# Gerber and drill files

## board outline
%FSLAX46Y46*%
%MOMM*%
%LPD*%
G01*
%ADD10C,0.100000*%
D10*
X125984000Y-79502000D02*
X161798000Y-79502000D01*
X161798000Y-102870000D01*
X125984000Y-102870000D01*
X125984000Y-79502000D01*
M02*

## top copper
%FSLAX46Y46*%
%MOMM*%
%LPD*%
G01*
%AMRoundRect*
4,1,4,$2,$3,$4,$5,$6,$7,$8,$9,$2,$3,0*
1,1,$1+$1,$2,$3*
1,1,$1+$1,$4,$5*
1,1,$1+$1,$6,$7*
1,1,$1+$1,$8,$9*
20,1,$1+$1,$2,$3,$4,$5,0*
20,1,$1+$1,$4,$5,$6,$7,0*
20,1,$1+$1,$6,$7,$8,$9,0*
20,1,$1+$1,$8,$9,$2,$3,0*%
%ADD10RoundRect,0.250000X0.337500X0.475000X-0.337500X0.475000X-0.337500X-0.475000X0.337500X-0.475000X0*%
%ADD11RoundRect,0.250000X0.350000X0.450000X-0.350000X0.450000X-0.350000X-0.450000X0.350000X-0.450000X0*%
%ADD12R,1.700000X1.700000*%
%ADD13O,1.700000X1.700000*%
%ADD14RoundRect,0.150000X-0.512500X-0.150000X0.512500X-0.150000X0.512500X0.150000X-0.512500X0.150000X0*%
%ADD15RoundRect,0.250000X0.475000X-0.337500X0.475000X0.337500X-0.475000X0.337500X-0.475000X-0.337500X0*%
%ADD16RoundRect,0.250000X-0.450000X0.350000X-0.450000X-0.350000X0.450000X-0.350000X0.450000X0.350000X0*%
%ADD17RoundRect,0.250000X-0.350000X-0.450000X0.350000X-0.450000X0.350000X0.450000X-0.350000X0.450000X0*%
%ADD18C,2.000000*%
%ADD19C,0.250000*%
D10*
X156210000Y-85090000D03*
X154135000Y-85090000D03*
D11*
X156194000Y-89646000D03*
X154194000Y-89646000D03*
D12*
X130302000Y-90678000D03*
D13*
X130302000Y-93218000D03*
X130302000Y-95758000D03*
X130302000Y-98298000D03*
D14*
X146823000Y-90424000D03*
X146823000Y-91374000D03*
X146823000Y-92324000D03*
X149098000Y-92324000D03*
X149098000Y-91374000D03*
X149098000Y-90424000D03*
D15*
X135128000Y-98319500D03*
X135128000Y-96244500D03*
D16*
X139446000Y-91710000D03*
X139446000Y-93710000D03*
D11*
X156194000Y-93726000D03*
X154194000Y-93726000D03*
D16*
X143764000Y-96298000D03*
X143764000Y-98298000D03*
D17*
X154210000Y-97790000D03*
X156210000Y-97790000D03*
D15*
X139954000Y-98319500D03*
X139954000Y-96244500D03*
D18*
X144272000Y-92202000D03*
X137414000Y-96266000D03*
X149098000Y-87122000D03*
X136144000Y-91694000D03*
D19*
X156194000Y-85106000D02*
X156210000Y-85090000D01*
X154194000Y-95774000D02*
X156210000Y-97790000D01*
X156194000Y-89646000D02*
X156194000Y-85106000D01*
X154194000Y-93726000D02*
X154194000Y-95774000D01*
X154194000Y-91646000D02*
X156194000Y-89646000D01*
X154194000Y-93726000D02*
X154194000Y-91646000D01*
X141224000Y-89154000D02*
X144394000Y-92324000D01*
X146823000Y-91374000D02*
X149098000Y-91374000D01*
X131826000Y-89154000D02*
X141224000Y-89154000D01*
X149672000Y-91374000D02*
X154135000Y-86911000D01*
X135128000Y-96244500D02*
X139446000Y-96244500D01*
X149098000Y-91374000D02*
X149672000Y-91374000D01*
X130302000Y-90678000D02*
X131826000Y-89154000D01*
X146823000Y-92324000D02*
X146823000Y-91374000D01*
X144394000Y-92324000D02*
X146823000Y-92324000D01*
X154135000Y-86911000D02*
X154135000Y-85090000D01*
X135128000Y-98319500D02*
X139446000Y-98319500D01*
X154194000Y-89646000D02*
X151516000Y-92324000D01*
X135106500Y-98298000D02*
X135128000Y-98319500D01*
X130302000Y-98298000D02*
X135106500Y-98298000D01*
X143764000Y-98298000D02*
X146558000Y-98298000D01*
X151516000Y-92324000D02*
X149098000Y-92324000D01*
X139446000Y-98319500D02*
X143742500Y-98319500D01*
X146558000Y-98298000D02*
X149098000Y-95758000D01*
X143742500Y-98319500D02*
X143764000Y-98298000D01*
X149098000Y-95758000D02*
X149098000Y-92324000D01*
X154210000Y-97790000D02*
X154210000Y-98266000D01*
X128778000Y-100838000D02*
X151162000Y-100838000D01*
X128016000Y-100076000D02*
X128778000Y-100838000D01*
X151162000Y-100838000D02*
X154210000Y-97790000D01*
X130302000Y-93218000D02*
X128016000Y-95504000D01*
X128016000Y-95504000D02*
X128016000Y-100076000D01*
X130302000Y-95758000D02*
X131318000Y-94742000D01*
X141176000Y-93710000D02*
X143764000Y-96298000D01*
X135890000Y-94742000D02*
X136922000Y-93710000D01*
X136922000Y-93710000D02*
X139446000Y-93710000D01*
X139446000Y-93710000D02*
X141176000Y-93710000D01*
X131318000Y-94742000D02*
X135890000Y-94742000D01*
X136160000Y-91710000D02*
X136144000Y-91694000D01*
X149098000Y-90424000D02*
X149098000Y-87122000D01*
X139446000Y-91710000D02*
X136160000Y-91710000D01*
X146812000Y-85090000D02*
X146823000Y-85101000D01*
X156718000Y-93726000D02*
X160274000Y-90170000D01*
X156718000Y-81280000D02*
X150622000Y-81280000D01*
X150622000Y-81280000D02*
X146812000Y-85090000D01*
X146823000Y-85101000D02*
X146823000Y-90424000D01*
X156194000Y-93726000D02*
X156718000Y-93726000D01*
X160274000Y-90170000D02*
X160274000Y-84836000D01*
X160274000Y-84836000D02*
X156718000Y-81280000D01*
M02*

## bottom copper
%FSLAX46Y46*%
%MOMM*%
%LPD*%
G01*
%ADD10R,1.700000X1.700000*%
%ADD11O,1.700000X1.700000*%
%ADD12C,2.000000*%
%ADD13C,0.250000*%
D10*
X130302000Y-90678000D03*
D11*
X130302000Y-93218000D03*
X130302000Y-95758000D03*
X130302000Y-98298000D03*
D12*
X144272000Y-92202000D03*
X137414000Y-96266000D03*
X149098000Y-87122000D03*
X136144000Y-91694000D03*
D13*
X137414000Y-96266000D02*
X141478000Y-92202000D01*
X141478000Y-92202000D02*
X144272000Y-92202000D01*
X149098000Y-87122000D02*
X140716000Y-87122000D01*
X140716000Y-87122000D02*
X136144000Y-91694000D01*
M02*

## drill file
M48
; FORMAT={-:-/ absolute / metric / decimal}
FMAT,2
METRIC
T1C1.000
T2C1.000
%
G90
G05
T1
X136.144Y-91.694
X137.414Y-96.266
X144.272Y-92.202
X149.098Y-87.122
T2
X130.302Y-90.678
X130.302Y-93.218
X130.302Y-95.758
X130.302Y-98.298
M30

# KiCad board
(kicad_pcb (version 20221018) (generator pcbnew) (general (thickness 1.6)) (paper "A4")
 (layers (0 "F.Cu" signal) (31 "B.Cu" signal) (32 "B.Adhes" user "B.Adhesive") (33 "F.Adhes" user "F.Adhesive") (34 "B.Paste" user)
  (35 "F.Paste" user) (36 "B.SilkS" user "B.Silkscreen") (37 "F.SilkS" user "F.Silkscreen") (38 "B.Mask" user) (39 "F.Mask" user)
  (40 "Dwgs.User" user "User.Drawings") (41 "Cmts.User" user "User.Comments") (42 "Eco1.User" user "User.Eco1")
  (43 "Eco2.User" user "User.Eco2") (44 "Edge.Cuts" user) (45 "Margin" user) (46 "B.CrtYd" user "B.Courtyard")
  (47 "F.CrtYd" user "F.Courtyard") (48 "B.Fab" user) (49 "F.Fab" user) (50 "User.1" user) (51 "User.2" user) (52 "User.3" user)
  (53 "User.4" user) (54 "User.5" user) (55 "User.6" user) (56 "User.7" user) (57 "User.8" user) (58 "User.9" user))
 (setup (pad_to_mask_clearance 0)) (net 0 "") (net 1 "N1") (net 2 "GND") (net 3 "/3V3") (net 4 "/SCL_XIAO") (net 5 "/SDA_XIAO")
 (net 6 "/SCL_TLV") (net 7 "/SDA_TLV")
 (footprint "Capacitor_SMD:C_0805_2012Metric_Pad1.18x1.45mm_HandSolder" (layer "F.Cu") (at 155.1725 85.09 180)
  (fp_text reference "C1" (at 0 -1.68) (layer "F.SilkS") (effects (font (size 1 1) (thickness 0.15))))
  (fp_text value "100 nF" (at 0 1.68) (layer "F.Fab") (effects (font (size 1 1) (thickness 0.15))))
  (pad "1" smd roundrect (at -1.0375 0 180) (size 1.175 1.45) (layers "F.Cu" "F.Paste" "F.Mask") (roundrect_rratio 0.2127659574)
   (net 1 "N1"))
  (pad "2" smd roundrect (at 1.0375 0 180) (size 1.175 1.45) (layers "F.Cu" "F.Paste" "F.Mask") (roundrect_rratio 0.2127659574)
   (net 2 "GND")))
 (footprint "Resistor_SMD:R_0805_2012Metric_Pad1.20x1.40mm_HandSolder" (layer "F.Cu") (at 155.194 89.646 180)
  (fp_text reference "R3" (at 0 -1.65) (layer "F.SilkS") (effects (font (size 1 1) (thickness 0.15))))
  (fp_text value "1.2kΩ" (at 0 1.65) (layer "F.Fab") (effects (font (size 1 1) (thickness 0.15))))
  (pad "1" smd roundrect (at -1 0 180) (size 1.2 1.4) (layers "F.Cu" "F.Paste" "F.Mask") (roundrect_rratio 0.2083333333) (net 1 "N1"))
  (pad "2" smd roundrect (at 1 0 180) (size 1.2 1.4) (layers "F.Cu" "F.Paste" "F.Mask") (roundrect_rratio 0.2083333333) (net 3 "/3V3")))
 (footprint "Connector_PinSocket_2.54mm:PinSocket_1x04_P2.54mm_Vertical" (layer "F.Cu") (at 130.302 90.678)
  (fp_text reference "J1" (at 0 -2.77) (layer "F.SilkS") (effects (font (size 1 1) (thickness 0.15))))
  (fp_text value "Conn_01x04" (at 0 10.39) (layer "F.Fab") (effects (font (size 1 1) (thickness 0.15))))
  (pad "1" thru_hole rect (at 0 0) (size 1.7 1.7) (drill 1) (layers "*.Cu" "*.Mask") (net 2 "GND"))
  (pad "2" thru_hole oval (at 0 2.54) (size 1.7 1.7) (drill 1) (layers "*.Cu" "*.Mask") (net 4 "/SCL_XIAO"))
  (pad "3" thru_hole oval (at 0 5.08) (size 1.7 1.7) (drill 1) (layers "*.Cu" "*.Mask") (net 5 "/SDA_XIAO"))
  (pad "4" thru_hole oval (at 0 7.62) (size 1.7 1.7) (drill 1) (layers "*.Cu" "*.Mask") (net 3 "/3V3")))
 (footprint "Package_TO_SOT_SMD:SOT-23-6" (layer "F.Cu") (at 147.9605 91.374)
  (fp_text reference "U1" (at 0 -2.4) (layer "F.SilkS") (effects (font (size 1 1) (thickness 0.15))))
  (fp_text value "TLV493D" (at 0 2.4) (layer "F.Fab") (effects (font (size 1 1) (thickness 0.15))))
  (pad "1" smd roundrect (at -1.1375 -0.95) (size 1.325 0.6) (layers "F.Cu" "F.Paste" "F.Mask") (roundrect_rratio 0.25) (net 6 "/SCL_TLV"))
  (pad "2" smd roundrect (at -1.1375 0) (size 1.325 0.6) (layers "F.Cu" "F.Paste" "F.Mask") (roundrect_rratio 0.25) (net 2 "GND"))
  (pad "3" smd roundrect (at -1.1375 0.95) (size 1.325 0.6) (layers "F.Cu" "F.Paste" "F.Mask") (roundrect_rratio 0.25) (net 2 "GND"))
  (pad "4" smd roundrect (at 1.1375 0.95) (size 1.325 0.6) (layers "F.Cu" "F.Paste" "F.Mask") (roundrect_rratio 0.25) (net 3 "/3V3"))
  (pad "5" smd roundrect (at 1.1375 0) (size 1.325 0.6) (layers "F.Cu" "F.Paste" "F.Mask") (roundrect_rratio 0.25) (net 2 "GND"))
  (pad "6" smd roundrect (at 1.1375 -0.95) (size 1.325 0.6) (layers "F.Cu" "F.Paste" "F.Mask") (roundrect_rratio 0.25) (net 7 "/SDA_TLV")))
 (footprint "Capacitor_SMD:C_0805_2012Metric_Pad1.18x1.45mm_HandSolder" (layer "F.Cu") (at 135.128 97.282 90)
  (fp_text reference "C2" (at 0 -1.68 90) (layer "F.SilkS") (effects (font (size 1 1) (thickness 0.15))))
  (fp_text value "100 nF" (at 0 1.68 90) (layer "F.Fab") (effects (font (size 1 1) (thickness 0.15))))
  (pad "1" smd roundrect (at -1.0375 0 90) (size 1.175 1.45) (layers "F.Cu" "F.Paste" "F.Mask") (roundrect_rratio 0.2127659574)
   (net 3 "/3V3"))
  (pad "2" smd roundrect (at 1.0375 0 90) (size 1.175 1.45) (layers "F.Cu" "F.Paste" "F.Mask") (roundrect_rratio 0.2127659574) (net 2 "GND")))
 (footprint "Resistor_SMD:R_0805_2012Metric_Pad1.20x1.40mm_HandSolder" (layer "F.Cu") (at 139.446 92.71 -90)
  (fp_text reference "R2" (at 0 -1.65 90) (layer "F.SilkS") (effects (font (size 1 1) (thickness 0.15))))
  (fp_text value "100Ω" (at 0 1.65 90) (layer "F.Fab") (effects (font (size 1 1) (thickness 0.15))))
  (pad "1" smd roundrect (at -1 0 270) (size 1.2 1.4) (layers "F.Cu" "F.Paste" "F.Mask") (roundrect_rratio 0.2083333333) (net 7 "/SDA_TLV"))
  (pad "2" smd roundrect (at 1 0 270) (size 1.2 1.4) (layers "F.Cu" "F.Paste" "F.Mask") (roundrect_rratio 0.2083333333) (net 5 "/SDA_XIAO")))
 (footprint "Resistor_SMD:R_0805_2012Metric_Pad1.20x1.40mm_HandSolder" (layer "F.Cu") (at 155.194 93.726 180)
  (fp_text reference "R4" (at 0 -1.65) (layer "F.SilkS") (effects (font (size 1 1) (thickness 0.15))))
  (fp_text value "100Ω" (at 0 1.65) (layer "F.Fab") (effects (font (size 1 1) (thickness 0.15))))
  (pad "1" smd roundrect (at -1 0 180) (size 1.2 1.4) (layers "F.Cu" "F.Paste" "F.Mask") (roundrect_rratio 0.2083333333) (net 6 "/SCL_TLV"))
  (pad "2" smd roundrect (at 1 0 180) (size 1.2 1.4) (layers "F.Cu" "F.Paste" "F.Mask") (roundrect_rratio 0.2083333333) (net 1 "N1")))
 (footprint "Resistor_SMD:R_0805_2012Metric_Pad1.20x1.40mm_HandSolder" (layer "F.Cu") (at 143.764 97.298 -90)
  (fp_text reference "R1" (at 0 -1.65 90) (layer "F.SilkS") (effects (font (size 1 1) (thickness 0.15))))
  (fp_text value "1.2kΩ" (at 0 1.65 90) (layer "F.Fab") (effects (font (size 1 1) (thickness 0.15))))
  (pad "1" smd roundrect (at -1 0 270) (size 1.2 1.4) (layers "F.Cu" "F.Paste" "F.Mask") (roundrect_rratio 0.2083333333) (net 5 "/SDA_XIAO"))
  (pad "2" smd roundrect (at 1 0 270) (size 1.2 1.4) (layers "F.Cu" "F.Paste" "F.Mask") (roundrect_rratio 0.2083333333) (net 3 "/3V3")))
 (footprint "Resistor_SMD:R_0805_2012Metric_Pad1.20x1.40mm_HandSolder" (layer "F.Cu") (at 155.21 97.79)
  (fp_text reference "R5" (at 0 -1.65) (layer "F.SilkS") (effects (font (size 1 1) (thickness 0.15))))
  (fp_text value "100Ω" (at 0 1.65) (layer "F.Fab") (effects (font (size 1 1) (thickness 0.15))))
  (pad "1" smd roundrect (at -1 0) (size 1.2 1.4) (layers "F.Cu" "F.Paste" "F.Mask") (roundrect_rratio 0.2083333333) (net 4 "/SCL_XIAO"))
  (pad "2" smd roundrect (at 1 0) (size 1.2 1.4) (layers "F.Cu" "F.Paste" "F.Mask") (roundrect_rratio 0.2083333333) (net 1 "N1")))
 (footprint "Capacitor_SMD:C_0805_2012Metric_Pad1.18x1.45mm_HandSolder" (layer "F.Cu") (at 139.954 97.282 90)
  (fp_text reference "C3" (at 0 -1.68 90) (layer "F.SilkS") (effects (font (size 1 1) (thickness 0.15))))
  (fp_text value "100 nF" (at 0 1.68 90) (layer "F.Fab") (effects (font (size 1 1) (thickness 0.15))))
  (pad "1" smd roundrect (at -1.0375 0 90) (size 1.175 1.45) (layers "F.Cu" "F.Paste" "F.Mask") (roundrect_rratio 0.2127659574)
   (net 3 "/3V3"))
  (pad "2" smd roundrect (at 1.0375 0 90) (size 1.175 1.45) (layers "F.Cu" "F.Paste" "F.Mask") (roundrect_rratio 0.2127659574) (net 2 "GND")))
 (gr_rect (start 125.984 79.502) (end 161.798 102.87) (stroke (width 0.1) (type default)) (fill none) (layer "Edge.Cuts"))
 (segment (start 156.194 85.106) (end 156.21 85.09) (width 0.25) (layer "F.Cu") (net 1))
 (segment (start 154.194 95.774) (end 156.21 97.79) (width 0.25) (layer "F.Cu") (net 1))
 (segment (start 156.194 89.646) (end 156.194 85.106) (width 0.25) (layer "F.Cu") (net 1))
 (segment (start 154.194 93.726) (end 154.194 95.774) (width 0.25) (layer "F.Cu") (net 1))
 (segment (start 154.194 91.646) (end 156.194 89.646) (width 0.25) (layer "F.Cu") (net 1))
 (segment (start 154.194 93.726) (end 154.194 91.646) (width 0.25) (layer "F.Cu") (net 1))
 (segment (start 141.224 89.154) (end 144.394 92.324) (width 0.25) (layer "F.Cu") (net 2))
 (segment (start 146.823 91.374) (end 149.098 91.374) (width 0.25) (layer "F.Cu") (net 2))
 (segment (start 131.826 89.154) (end 141.224 89.154) (width 0.25) (layer "F.Cu") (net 2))
 (segment (start 149.672 91.374) (end 154.135 86.911) (width 0.25) (layer "F.Cu") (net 2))
 (segment (start 135.128 96.2445) (end 139.446 96.2445) (width 0.25) (layer "F.Cu") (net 2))
 (segment (start 149.098 91.374) (end 149.672 91.374) (width 0.25) (layer "F.Cu") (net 2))
 (segment (start 130.302 90.678) (end 131.826 89.154) (width 0.25) (layer "F.Cu") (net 2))
 (segment (start 146.823 92.324) (end 146.823 91.374) (width 0.25) (layer "F.Cu") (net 2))
 (segment (start 144.394 92.324) (end 146.823 92.324) (width 0.25) (layer "F.Cu") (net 2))
 (segment (start 154.135 86.911) (end 154.135 85.09) (width 0.25) (layer "F.Cu") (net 2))
 (via (at 144.272 92.202) (size 2) (drill 1) (layers "F.Cu" "B.Cu") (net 2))
 (via (at 137.414 96.266) (size 2) (drill 1) (layers "F.Cu" "B.Cu") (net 2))
 (segment (start 137.414 96.266) (end 141.478 92.202) (width 0.25) (layer "B.Cu") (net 2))
 (segment (start 141.478 92.202) (end 144.272 92.202) (width 0.25) (layer "B.Cu") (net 2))
 (segment (start 135.128 98.3195) (end 139.446 98.3195) (width 0.25) (layer "F.Cu") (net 3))
 (segment (start 154.194 89.646) (end 151.516 92.324) (width 0.25) (layer "F.Cu") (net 3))
 (segment (start 135.1065 98.298) (end 135.128 98.3195) (width 0.25) (layer "F.Cu") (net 3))
 (segment (start 130.302 98.298) (end 135.1065 98.298) (width 0.25) (layer "F.Cu") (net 3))
 (segment (start 143.764 98.298) (end 146.558 98.298) (width 0.25) (layer "F.Cu") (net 3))
 (segment (start 151.516 92.324) (end 149.098 92.324) (width 0.25) (layer "F.Cu") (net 3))
 (segment (start 139.446 98.3195) (end 143.7425 98.3195) (width 0.25) (layer "F.Cu") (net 3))
 (segment (start 146.558 98.298) (end 149.098 95.758) (width 0.25) (layer "F.Cu") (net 3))
 (segment (start 143.7425 98.3195) (end 143.764 98.298) (width 0.25) (layer "F.Cu") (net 3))
 (segment (start 149.098 95.758) (end 149.098 92.324) (width 0.25) (layer "F.Cu") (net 3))
 (segment (start 154.21 97.79) (end 154.21 98.266) (width 0.25) (layer "F.Cu") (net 4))
 (segment (start 128.778 100.838) (end 151.162 100.838) (width 0.25) (layer "F.Cu") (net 4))
 (segment (start 128.016 100.076) (end 128.778 100.838) (width 0.25) (layer "F.Cu") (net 4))
 (segment (start 151.162 100.838) (end 154.21 97.79) (width 0.25) (layer "F.Cu") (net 4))
 (segment (start 130.302 93.218) (end 128.016 95.504) (width 0.25) (layer "F.Cu") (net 4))
 (segment (start 128.016 95.504) (end 128.016 100.076) (width 0.25) (layer "F.Cu") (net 4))
 (segment (start 130.302 95.758) (end 131.318 94.742) (width 0.25) (layer "F.Cu") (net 5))
 (segment (start 141.176 93.71) (end 143.764 96.298) (width 0.25) (layer "F.Cu") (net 5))
 (segment (start 135.89 94.742) (end 136.922 93.71) (width 0.25) (layer "F.Cu") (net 5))
 (segment (start 136.922 93.71) (end 139.446 93.71) (width 0.25) (layer "F.Cu") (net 5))
 (segment (start 139.446 93.71) (end 141.176 93.71) (width 0.25) (layer "F.Cu") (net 5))
 (segment (start 131.318 94.742) (end 135.89 94.742) (width 0.25) (layer "F.Cu") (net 5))
 (segment (start 136.16 91.71) (end 136.144 91.694) (width 0.25) (layer "F.Cu") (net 7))
 (segment (start 149.098 90.424) (end 149.098 87.122) (width 0.25) (layer "F.Cu") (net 7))
 (segment (start 139.446 91.71) (end 136.16 91.71) (width 0.25) (layer "F.Cu") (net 7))
 (via (at 149.098 87.122) (size 2) (drill 1) (layers "F.Cu" "B.Cu") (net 7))
 (via (at 136.144 91.694) (size 2) (drill 1) (layers "F.Cu" "B.Cu") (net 7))
 (segment (start 149.098 87.122) (end 140.716 87.122) (width 0.25) (layer "B.Cu") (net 7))
 (segment (start 140.716 87.122) (end 136.144 91.694) (width 0.25) (layer "B.Cu") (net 7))
 (segment (start 146.812 85.09) (end 146.823 85.101) (width 0.25) (layer "F.Cu") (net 6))
 (segment (start 156.718 93.726) (end 160.274 90.17) (width 0.25) (layer "F.Cu") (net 6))
 (segment (start 156.718 81.28) (end 150.622 81.28) (width 0.25) (layer "F.Cu") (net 6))
 (segment (start 150.622 81.28) (end 146.812 85.09) (width 0.25) (layer "F.Cu") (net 6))
 (segment (start 146.823 85.101) (end 146.823 90.424) (width 0.25) (layer "F.Cu") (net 6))
 (segment (start 156.194 93.726) (end 156.718 93.726) (width 0.25) (layer "F.Cu") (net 6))
 (segment (start 160.274 90.17) (end 160.274 84.836) (width 0.25) (layer "F.Cu") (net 6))
 (segment (start 160.274 84.836) (end 156.718 81.28) (width 0.25) (layer "F.Cu") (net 6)))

